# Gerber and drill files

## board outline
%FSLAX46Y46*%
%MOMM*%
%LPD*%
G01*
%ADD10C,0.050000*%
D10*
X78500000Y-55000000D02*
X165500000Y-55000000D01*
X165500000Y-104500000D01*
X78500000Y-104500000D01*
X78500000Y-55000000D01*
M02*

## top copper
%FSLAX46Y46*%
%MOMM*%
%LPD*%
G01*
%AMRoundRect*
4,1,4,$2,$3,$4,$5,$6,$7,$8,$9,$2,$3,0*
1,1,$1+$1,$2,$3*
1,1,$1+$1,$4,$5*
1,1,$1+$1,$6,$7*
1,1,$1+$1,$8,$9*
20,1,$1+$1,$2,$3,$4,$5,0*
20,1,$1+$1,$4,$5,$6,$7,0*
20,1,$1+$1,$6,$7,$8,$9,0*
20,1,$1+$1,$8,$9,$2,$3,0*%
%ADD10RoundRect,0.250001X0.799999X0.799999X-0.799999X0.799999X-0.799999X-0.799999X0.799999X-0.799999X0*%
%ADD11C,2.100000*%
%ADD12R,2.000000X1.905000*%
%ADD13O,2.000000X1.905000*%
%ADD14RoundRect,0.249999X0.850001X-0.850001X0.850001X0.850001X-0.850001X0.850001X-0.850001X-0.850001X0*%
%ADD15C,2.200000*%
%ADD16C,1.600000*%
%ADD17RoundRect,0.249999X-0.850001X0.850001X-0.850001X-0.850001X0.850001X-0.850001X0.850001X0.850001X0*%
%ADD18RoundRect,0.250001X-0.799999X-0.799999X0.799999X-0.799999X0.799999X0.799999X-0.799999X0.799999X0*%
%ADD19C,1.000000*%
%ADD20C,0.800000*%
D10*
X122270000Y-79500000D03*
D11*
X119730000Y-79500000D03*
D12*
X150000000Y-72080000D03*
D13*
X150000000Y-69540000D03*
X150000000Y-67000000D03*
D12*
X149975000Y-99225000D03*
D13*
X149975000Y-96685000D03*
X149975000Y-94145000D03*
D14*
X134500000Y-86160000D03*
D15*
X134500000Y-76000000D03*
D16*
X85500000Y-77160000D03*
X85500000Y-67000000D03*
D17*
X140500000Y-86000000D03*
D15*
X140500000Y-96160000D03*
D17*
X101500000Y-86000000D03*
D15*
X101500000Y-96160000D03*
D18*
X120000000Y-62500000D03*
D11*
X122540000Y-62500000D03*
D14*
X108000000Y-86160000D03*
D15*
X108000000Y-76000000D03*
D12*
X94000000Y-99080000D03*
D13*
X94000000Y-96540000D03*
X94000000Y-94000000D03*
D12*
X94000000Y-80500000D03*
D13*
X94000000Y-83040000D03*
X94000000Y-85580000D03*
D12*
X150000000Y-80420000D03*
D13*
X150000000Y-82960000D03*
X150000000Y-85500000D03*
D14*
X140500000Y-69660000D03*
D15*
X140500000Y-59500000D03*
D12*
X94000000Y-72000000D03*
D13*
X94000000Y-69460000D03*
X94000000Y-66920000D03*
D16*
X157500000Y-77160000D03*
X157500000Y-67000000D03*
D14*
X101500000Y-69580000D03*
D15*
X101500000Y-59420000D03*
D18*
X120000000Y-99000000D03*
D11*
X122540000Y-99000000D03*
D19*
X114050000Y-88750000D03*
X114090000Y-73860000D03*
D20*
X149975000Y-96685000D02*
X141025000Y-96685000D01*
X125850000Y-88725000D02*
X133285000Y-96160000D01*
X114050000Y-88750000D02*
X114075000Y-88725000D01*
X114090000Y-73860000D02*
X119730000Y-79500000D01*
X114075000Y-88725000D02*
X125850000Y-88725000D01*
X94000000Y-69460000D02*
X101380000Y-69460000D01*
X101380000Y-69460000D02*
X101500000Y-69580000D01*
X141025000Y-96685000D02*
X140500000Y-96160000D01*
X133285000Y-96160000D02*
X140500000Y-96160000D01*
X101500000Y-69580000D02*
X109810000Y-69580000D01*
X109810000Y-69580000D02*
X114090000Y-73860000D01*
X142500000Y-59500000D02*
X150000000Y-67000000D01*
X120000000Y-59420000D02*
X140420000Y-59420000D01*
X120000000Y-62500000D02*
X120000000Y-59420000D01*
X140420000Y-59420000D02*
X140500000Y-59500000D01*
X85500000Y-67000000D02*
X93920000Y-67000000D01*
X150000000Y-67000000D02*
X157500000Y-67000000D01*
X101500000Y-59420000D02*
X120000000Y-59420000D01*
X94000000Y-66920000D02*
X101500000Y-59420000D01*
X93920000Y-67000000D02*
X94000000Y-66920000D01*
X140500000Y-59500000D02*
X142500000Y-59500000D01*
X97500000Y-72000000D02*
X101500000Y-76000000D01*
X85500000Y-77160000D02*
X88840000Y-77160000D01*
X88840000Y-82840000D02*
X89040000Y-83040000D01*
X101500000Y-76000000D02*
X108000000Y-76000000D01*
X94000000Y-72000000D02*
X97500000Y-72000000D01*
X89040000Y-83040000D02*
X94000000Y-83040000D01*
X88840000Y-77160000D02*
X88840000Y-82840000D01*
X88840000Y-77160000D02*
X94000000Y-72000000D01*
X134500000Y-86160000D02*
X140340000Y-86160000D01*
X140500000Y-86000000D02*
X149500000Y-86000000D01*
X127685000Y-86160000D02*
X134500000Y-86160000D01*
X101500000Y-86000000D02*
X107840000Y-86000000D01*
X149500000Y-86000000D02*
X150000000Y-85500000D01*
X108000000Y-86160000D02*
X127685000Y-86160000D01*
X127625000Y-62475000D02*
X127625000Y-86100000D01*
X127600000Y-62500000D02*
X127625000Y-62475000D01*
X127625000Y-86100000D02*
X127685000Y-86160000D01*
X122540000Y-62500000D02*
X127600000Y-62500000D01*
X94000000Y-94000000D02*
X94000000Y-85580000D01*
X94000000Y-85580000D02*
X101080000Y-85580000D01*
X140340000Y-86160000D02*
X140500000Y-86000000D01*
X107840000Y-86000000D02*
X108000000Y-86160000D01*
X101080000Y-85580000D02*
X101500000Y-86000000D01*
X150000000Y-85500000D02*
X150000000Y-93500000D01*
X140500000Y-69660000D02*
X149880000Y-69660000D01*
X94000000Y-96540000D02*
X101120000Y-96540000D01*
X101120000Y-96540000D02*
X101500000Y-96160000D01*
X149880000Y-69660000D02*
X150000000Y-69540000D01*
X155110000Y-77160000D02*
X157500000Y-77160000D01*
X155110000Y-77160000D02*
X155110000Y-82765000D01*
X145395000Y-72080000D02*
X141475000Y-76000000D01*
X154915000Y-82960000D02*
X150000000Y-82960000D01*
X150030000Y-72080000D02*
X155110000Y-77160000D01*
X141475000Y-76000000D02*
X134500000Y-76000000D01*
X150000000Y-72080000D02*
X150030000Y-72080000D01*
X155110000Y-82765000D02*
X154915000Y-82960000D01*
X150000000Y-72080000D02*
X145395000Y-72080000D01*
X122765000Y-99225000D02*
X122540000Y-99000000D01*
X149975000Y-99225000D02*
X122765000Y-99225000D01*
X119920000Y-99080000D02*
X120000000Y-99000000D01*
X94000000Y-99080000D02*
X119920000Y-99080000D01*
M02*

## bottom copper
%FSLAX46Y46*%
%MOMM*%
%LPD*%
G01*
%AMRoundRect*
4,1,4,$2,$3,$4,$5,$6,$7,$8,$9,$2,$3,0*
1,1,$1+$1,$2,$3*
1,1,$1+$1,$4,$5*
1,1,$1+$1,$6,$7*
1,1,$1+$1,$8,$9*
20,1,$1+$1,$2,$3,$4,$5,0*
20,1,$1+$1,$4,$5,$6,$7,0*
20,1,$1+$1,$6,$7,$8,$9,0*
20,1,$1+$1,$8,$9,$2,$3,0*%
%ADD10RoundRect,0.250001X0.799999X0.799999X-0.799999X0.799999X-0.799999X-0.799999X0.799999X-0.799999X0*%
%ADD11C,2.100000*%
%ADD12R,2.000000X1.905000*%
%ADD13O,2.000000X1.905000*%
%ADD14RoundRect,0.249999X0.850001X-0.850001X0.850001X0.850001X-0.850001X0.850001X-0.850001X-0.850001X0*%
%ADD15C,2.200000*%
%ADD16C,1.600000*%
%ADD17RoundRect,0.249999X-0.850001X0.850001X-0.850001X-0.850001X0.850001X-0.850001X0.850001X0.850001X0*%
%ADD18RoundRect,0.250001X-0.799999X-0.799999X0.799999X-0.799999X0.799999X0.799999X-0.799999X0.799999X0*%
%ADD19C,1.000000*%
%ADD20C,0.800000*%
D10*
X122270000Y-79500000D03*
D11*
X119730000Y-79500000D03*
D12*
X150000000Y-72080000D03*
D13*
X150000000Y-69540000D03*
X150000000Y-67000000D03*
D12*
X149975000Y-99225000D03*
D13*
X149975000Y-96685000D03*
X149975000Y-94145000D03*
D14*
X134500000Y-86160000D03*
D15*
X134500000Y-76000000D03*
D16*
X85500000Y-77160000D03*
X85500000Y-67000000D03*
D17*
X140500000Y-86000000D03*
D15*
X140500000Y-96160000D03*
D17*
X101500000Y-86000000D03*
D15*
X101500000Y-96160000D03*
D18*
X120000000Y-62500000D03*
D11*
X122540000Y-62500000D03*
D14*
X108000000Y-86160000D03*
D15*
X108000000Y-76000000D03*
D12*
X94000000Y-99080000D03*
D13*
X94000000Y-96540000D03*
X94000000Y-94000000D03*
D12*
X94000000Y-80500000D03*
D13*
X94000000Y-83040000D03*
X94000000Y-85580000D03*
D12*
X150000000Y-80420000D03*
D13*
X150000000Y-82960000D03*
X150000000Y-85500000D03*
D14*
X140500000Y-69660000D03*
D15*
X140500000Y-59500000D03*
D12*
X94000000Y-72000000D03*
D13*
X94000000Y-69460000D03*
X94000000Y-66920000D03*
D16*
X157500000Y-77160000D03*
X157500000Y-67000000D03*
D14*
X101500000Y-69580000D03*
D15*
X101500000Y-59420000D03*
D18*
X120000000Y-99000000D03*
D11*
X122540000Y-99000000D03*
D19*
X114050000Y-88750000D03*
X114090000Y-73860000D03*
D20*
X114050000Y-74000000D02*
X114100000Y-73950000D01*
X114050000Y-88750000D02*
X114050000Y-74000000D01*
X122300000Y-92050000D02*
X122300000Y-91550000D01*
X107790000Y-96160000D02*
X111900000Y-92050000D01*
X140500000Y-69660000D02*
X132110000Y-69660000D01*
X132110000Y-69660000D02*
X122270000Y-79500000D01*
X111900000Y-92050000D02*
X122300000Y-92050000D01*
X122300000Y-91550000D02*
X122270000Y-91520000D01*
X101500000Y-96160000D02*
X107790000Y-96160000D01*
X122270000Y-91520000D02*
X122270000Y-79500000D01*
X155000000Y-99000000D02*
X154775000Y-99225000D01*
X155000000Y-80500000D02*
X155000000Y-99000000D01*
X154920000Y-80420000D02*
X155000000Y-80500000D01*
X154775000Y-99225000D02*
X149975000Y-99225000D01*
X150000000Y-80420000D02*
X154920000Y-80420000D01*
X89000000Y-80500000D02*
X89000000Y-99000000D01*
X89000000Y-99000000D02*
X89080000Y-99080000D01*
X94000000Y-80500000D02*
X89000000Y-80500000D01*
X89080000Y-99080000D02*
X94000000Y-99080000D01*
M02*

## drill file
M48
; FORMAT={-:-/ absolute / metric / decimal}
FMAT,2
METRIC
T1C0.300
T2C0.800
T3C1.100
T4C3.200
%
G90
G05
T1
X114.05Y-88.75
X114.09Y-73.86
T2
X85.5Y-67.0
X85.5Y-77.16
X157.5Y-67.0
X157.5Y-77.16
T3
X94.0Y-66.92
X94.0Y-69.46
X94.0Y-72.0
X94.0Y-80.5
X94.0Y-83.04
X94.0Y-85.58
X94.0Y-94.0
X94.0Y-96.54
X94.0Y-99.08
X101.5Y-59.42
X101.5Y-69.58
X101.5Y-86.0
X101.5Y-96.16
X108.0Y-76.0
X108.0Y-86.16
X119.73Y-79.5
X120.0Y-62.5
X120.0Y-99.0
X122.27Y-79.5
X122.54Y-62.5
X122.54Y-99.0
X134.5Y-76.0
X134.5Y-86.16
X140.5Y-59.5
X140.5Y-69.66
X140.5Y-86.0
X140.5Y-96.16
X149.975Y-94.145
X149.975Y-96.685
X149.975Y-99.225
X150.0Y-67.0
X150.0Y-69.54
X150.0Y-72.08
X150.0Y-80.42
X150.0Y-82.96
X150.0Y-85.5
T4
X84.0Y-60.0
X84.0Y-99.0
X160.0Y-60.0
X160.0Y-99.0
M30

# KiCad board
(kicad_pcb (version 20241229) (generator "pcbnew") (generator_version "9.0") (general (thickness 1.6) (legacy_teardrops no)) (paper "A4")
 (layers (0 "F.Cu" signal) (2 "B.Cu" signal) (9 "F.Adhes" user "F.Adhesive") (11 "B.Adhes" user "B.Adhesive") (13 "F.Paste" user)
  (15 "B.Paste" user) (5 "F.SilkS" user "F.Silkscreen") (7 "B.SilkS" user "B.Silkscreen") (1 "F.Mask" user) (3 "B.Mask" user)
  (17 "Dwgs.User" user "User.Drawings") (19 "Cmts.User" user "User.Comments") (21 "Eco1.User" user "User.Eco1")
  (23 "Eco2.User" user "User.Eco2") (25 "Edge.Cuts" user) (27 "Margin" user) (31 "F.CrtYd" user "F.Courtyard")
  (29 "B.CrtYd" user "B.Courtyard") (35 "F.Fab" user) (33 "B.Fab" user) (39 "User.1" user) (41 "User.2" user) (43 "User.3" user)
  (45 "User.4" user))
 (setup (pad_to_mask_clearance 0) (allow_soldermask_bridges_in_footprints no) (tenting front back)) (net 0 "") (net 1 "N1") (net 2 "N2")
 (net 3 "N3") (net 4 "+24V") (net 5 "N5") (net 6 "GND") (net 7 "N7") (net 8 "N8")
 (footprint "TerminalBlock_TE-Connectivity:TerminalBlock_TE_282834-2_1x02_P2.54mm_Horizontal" (layer "F.Cu") (at 122.27 79.5 180)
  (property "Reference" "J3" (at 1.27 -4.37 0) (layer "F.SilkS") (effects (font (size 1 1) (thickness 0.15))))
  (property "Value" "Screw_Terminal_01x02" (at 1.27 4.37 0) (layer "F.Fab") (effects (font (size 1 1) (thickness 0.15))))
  (pad "1" thru_hole roundrect (at 0 0 180) (size 2.1 2.1) (drill 1.1) (layers "*.Cu" "*.Mask") (remove_unused_layers no)
   (roundrect_rratio 0.119048) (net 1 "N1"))
  (pad "2" thru_hole circle (at 2.54 0 180) (size 2.1 2.1) (drill 1.1) (layers "*.Cu" "*.Mask") (remove_unused_layers no) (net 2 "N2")))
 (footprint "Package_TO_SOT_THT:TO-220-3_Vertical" (layer "F.Cu") (at 150 72.08 90)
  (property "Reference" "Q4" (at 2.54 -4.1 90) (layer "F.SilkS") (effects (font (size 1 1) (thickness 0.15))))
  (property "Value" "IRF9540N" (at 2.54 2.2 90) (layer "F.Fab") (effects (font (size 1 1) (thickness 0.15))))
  (pad "1" thru_hole rect (at 0 0 90) (size 1.905 2) (drill 1.1) (layers "*.Cu" "*.Mask") (remove_unused_layers no) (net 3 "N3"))
  (pad "2" thru_hole oval (at 2.54 0 90) (size 1.905 2) (drill 1.1) (layers "*.Cu" "*.Mask") (remove_unused_layers no) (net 1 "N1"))
  (pad "3" thru_hole oval (at 5.08 0 90) (size 1.905 2) (drill 1.1) (layers "*.Cu" "*.Mask") (remove_unused_layers no) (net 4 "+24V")))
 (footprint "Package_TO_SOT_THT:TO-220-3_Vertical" (layer "F.Cu") (at 149.975 99.225 90)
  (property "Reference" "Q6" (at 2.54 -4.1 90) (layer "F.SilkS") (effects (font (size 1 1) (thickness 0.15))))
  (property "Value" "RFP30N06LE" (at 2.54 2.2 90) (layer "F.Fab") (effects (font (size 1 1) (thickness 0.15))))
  (pad "1" thru_hole rect (at 0 0 90) (size 1.905 2) (drill 1.1) (layers "*.Cu" "*.Mask") (remove_unused_layers no) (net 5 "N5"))
  (pad "2" thru_hole oval (at 2.54 0 90) (size 1.905 2) (drill 1.1) (layers "*.Cu" "*.Mask") (remove_unused_layers no) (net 2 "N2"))
  (pad "3" thru_hole oval (at 5.08 0 90) (size 1.905 2) (drill 1.1) (layers "*.Cu" "*.Mask") (remove_unused_layers no) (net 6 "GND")))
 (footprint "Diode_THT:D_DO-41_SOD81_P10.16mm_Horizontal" (layer "F.Cu") (at 134.5 86.16 90)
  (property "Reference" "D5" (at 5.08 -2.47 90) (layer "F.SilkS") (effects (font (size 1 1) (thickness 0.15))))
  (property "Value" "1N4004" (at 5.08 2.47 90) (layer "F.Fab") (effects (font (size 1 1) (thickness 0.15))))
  (pad "1" thru_hole roundrect (at 0 0 90) (size 2.2 2.2) (drill 1.1) (layers "*.Cu" "*.Mask") (remove_unused_layers no)
   (roundrect_rratio 0.113636) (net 6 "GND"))
  (pad "2" thru_hole circle (at 10.16 0 90) (size 2.2 2.2) (drill 1.1) (layers "*.Cu" "*.Mask") (remove_unused_layers no) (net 3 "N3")))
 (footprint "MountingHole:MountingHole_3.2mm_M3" (layer "F.Cu") (at 84 99)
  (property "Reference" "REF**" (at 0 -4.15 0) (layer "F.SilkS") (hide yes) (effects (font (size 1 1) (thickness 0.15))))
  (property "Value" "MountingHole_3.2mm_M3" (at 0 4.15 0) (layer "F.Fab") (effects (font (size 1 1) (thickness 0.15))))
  (pad "" np_thru_hole circle (at 0 0) (size 3.2 3.2) (drill 3.2) (layers "*.Cu" "*.Mask")))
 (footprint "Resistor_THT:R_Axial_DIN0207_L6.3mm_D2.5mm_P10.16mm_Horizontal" (layer "F.Cu") (at 85.5 77.16 90)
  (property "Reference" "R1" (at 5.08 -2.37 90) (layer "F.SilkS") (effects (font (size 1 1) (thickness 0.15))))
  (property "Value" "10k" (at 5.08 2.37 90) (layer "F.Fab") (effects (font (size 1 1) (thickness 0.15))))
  (pad "1" thru_hole circle (at 0 0 90) (size 1.6 1.6) (drill 0.8) (layers "*.Cu" "*.Mask") (remove_unused_layers no) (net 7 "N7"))
  (pad "2" thru_hole circle (at 10.16 0 90) (size 1.6 1.6) (drill 0.8) (layers "*.Cu" "*.Mask") (remove_unused_layers no) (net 4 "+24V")))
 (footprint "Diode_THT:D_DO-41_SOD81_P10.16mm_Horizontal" (layer "F.Cu") (at 140.5 86 -90)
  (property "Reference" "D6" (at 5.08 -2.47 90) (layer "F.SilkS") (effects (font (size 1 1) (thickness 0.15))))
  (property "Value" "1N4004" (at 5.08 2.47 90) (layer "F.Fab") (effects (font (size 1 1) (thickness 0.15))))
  (pad "1" thru_hole roundrect (at 0 0 270) (size 2.2 2.2) (drill 1.1) (layers "*.Cu" "*.Mask") (remove_unused_layers no)
   (roundrect_rratio 0.113636) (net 6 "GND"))
  (pad "2" thru_hole circle (at 10.16 0 270) (size 2.2 2.2) (drill 1.1) (layers "*.Cu" "*.Mask") (remove_unused_layers no) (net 2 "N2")))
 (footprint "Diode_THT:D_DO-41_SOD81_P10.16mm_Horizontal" (layer "F.Cu") (at 101.5 86 -90)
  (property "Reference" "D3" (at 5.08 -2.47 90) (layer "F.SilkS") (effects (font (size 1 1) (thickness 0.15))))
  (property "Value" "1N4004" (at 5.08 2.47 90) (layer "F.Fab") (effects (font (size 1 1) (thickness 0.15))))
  (pad "1" thru_hole roundrect (at 0 0 270) (size 2.2 2.2) (drill 1.1) (layers "*.Cu" "*.Mask") (remove_unused_layers no)
   (roundrect_rratio 0.113636) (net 6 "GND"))
  (pad "2" thru_hole circle (at 10.16 0 270) (size 2.2 2.2) (drill 1.1) (layers "*.Cu" "*.Mask") (remove_unused_layers no) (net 1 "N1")))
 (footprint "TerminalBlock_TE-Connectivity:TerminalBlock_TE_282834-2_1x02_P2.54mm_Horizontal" (layer "F.Cu") (at 120 62.5)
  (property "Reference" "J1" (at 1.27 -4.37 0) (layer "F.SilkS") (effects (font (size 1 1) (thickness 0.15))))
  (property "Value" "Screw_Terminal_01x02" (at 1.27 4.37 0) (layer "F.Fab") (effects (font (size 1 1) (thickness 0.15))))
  (pad "1" thru_hole roundrect (at 0 0) (size 2.1 2.1) (drill 1.1) (layers "*.Cu" "*.Mask") (remove_unused_layers no)
   (roundrect_rratio 0.119048) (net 4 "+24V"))
  (pad "2" thru_hole circle (at 2.54 0) (size 2.1 2.1) (drill 1.1) (layers "*.Cu" "*.Mask") (remove_unused_layers no) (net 6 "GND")))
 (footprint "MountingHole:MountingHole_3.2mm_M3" (layer "F.Cu") (at 84 60)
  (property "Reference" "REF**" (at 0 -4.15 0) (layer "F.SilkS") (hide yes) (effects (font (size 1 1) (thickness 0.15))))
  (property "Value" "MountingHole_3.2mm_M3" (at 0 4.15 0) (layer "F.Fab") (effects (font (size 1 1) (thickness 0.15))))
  (pad "" np_thru_hole circle (at 0 0) (size 3.2 3.2) (drill 3.2) (layers "*.Cu" "*.Mask")))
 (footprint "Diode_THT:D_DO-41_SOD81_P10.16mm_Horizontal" (layer "F.Cu") (at 108 86.16 90)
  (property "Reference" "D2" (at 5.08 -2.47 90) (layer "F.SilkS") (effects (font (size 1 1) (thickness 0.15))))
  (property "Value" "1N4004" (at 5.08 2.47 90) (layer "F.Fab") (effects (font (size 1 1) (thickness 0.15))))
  (pad "1" thru_hole roundrect (at 0 0 90) (size 2.2 2.2) (drill 1.1) (layers "*.Cu" "*.Mask") (remove_unused_layers no)
   (roundrect_rratio 0.113636) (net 6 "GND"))
  (pad "2" thru_hole circle (at 10.16 0 90) (size 2.2 2.2) (drill 1.1) (layers "*.Cu" "*.Mask") (remove_unused_layers no) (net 7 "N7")))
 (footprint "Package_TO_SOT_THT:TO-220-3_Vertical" (layer "F.Cu") (at 94 99.08 90)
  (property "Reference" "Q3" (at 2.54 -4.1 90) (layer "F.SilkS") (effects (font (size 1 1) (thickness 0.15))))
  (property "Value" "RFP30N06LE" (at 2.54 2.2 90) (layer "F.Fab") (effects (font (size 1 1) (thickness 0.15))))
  (pad "1" thru_hole rect (at 0 0 90) (size 1.905 2) (drill 1.1) (layers "*.Cu" "*.Mask") (remove_unused_layers no) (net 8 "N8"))
  (pad "2" thru_hole oval (at 2.54 0 90) (size 1.905 2) (drill 1.1) (layers "*.Cu" "*.Mask") (remove_unused_layers no) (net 1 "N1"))
  (pad "3" thru_hole oval (at 5.08 0 90) (size 1.905 2) (drill 1.1) (layers "*.Cu" "*.Mask") (remove_unused_layers no) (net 6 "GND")))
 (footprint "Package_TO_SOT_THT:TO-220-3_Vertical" (layer "F.Cu") (at 94 80.5 -90)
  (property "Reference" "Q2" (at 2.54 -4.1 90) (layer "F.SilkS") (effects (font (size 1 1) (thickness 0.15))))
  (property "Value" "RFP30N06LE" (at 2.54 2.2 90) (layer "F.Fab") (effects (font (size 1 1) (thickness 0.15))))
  (pad "1" thru_hole rect (at 0 0 270) (size 1.905 2) (drill 1.1) (layers "*.Cu" "*.Mask") (remove_unused_layers no) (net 8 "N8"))
  (pad "2" thru_hole oval (at 2.54 0 270) (size 1.905 2) (drill 1.1) (layers "*.Cu" "*.Mask") (remove_unused_layers no) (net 7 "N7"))
  (pad "3" thru_hole oval (at 5.08 0 270) (size 1.905 2) (drill 1.1) (layers "*.Cu" "*.Mask") (remove_unused_layers no) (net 6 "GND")))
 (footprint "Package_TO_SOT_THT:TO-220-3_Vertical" (layer "F.Cu") (at 150 80.42 -90)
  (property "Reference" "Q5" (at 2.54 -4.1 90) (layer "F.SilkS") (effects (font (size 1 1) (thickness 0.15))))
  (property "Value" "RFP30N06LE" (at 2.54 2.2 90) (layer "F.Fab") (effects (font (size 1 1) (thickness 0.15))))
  (pad "1" thru_hole rect (at 0 0 270) (size 1.905 2) (drill 1.1) (layers "*.Cu" "*.Mask") (remove_unused_layers no) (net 5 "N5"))
  (pad "2" thru_hole oval (at 2.54 0 270) (size 1.905 2) (drill 1.1) (layers "*.Cu" "*.Mask") (remove_unused_layers no) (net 3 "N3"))
  (pad "3" thru_hole oval (at 5.08 0 270) (size 1.905 2) (drill 1.1) (layers "*.Cu" "*.Mask") (remove_unused_layers no) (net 6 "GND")))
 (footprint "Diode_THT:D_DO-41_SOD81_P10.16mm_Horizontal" (layer "F.Cu") (at 140.5 69.66 90)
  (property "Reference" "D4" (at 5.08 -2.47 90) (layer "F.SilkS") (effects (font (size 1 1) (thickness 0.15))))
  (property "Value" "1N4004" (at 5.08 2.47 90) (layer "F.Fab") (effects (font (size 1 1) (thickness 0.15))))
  (pad "1" thru_hole roundrect (at 0 0 90) (size 2.2 2.2) (drill 1.1) (layers "*.Cu" "*.Mask") (remove_unused_layers no)
   (roundrect_rratio 0.113636) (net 1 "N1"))
  (pad "2" thru_hole circle (at 10.16 0 90) (size 2.2 2.2) (drill 1.1) (layers "*.Cu" "*.Mask") (remove_unused_layers no) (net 4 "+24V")))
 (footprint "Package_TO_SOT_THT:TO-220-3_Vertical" (layer "F.Cu") (at 94 72 90)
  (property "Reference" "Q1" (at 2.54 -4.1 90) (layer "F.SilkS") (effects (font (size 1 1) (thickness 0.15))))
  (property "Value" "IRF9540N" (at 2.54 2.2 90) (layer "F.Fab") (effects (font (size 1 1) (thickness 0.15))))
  (pad "1" thru_hole rect (at 0 0 90) (size 1.905 2) (drill 1.1) (layers "*.Cu" "*.Mask") (remove_unused_layers no) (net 7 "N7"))
  (pad "2" thru_hole oval (at 2.54 0 90) (size 1.905 2) (drill 1.1) (layers "*.Cu" "*.Mask") (remove_unused_layers no) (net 2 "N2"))
  (pad "3" thru_hole oval (at 5.08 0 90) (size 1.905 2) (drill 1.1) (layers "*.Cu" "*.Mask") (remove_unused_layers no) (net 4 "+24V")))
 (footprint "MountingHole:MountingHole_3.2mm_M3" (layer "F.Cu") (at 160 60)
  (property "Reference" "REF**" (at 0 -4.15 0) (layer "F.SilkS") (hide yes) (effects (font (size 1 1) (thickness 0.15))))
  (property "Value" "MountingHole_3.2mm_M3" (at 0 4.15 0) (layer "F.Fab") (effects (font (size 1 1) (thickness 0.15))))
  (pad "" np_thru_hole circle (at 0 0) (size 3.2 3.2) (drill 3.2) (layers "*.Cu" "*.Mask")))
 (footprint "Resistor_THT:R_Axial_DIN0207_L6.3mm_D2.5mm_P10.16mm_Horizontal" (layer "F.Cu") (at 157.5 77.16 90)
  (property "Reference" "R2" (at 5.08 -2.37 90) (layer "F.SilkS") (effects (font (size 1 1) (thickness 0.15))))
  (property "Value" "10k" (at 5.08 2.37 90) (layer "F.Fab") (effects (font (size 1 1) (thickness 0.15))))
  (pad "1" thru_hole circle (at 0 0 90) (size 1.6 1.6) (drill 0.8) (layers "*.Cu" "*.Mask") (remove_unused_layers no) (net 3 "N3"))
  (pad "2" thru_hole circle (at 10.16 0 90) (size 1.6 1.6) (drill 0.8) (layers "*.Cu" "*.Mask") (remove_unused_layers no) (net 4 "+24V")))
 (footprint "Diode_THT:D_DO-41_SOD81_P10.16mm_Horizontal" (layer "F.Cu") (at 101.5 69.58 90)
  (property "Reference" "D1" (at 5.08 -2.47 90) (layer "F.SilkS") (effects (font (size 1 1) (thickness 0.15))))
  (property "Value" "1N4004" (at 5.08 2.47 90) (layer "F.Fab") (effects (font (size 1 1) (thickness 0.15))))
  (pad "1" thru_hole roundrect (at 0 0 90) (size 2.2 2.2) (drill 1.1) (layers "*.Cu" "*.Mask") (remove_unused_layers no)
   (roundrect_rratio 0.113636) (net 2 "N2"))
  (pad "2" thru_hole circle (at 10.16 0 90) (size 2.2 2.2) (drill 1.1) (layers "*.Cu" "*.Mask") (remove_unused_layers no) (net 4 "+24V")))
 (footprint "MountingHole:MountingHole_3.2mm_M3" (layer "F.Cu") (at 160 99)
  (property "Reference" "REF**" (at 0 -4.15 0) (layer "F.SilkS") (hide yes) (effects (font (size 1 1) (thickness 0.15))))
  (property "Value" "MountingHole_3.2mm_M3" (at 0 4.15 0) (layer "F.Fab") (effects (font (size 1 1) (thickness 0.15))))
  (pad "" np_thru_hole circle (at 0 0) (size 3.2 3.2) (drill 3.2) (layers "*.Cu" "*.Mask")))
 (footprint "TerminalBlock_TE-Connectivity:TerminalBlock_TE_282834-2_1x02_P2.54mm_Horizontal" (layer "F.Cu") (at 120 99)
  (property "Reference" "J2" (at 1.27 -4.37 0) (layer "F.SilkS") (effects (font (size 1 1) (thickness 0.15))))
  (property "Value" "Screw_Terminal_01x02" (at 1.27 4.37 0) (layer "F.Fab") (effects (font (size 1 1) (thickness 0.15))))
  (pad "1" thru_hole roundrect (at 0 0) (size 2.1 2.1) (drill 1.1) (layers "*.Cu" "*.Mask") (remove_unused_layers no)
   (roundrect_rratio 0.119048) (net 8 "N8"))
  (pad "2" thru_hole circle (at 2.54 0) (size 2.1 2.1) (drill 1.1) (layers "*.Cu" "*.Mask") (remove_unused_layers no) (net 5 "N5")))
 (gr_rect (start 78.5 55) (end 165.5 104.5) (stroke (width 0.05) (type default)) (fill no) (layer "Edge.Cuts"))
 (segment (start 149.975 96.685) (end 141.025 96.685) (width 0.8) (layer "F.Cu") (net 2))
 (segment (start 125.85 88.725) (end 133.285 96.16) (width 0.8) (layer "F.Cu") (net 2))
 (segment (start 114.05 88.75) (end 114.075 88.725) (width 0.8) (layer "F.Cu") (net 2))
 (segment (start 114.09 73.86) (end 119.73 79.5) (width 0.8) (layer "F.Cu") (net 2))
 (segment (start 114.075 88.725) (end 125.85 88.725) (width 0.8) (layer "F.Cu") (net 2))
 (segment (start 94 69.46) (end 101.38 69.46) (width 0.8) (layer "F.Cu") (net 2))
 (segment (start 101.38 69.46) (end 101.5 69.58) (width 0.8) (layer "F.Cu") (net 2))
 (segment (start 141.025 96.685) (end 140.5 96.16) (width 0.8) (layer "F.Cu") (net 2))
 (segment (start 133.285 96.16) (end 140.5 96.16) (width 0.8) (layer "F.Cu") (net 2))
 (segment (start 101.5 69.58) (end 109.81 69.58) (width 0.8) (layer "F.Cu") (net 2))
 (segment (start 109.81 69.58) (end 114.09 73.86) (width 0.8) (layer "F.Cu") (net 2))
 (via (at 114.05 88.75) (size 1) (drill 0.3) (layers "F.Cu" "B.Cu") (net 2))
 (via (at 114.09 73.86) (size 1) (drill 0.3) (layers "F.Cu" "B.Cu") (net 2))
 (segment (start 114.05 74) (end 114.1 73.95) (width 0.8) (layer "B.Cu") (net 2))
 (segment (start 114.05 88.75) (end 114.05 74) (width 0.8) (layer "B.Cu") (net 2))
 (segment (start 142.5 59.5) (end 150 67) (width 0.8) (layer "F.Cu") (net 4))
 (segment (start 120 59.42) (end 140.42 59.42) (width 0.8) (layer "F.Cu") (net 4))
 (segment (start 120 62.5) (end 120 59.42) (width 0.8) (layer "F.Cu") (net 4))
 (segment (start 140.42 59.42) (end 140.5 59.5) (width 0.8) (layer "F.Cu") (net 4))
 (segment (start 85.5 67) (end 93.92 67) (width 0.8) (layer "F.Cu") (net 4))
 (segment (start 150 67) (end 157.5 67) (width 0.8) (layer "F.Cu") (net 4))
 (segment (start 101.5 59.42) (end 120 59.42) (width 0.8) (layer "F.Cu") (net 4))
 (segment (start 94 66.92) (end 101.5 59.42) (width 0.8) (layer "F.Cu") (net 4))
 (segment (start 93.92 67) (end 94 66.92) (width 0.8) (layer "F.Cu") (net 4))
 (segment (start 140.5 59.5) (end 142.5 59.5) (width 0.8) (layer "F.Cu") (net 4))
 (segment (start 97.5 72) (end 101.5 76) (width 0.8) (layer "F.Cu") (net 7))
 (segment (start 85.5 77.16) (end 88.84 77.16) (width 0.8) (layer "F.Cu") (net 7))
 (segment (start 88.84 82.84) (end 89.04 83.04) (width 0.8) (layer "F.Cu") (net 7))
 (segment (start 101.5 76) (end 108 76) (width 0.8) (layer "F.Cu") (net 7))
 (segment (start 94 72) (end 97.5 72) (width 0.8) (layer "F.Cu") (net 7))
 (segment (start 89.04 83.04) (end 94 83.04) (width 0.8) (layer "F.Cu") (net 7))
 (segment (start 88.84 77.16) (end 88.84 82.84) (width 0.8) (layer "F.Cu") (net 7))
 (segment (start 88.84 77.16) (end 94 72) (width 0.8) (layer "F.Cu") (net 7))
 (segment (start 134.5 86.16) (end 140.34 86.16) (width 0.8) (layer "F.Cu") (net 6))
 (segment (start 140.5 86) (end 149.5 86) (width 0.8) (layer "F.Cu") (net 6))
 (segment (start 127.685 86.16) (end 134.5 86.16) (width 0.8) (layer "F.Cu") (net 6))
 (segment (start 101.5 86) (end 107.84 86) (width 0.8) (layer "F.Cu") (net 6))
 (segment (start 149.5 86) (end 150 85.5) (width 0.8) (layer "F.Cu") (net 6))
 (segment (start 108 86.16) (end 127.685 86.16) (width 0.8) (layer "F.Cu") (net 6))
 (segment (start 127.625 62.475) (end 127.625 86.1) (width 0.8) (layer "F.Cu") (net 6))
 (segment (start 127.6 62.5) (end 127.625 62.475) (width 0.8) (layer "F.Cu") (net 6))
 (segment (start 127.625 86.1) (end 127.685 86.16) (width 0.8) (layer "F.Cu") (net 6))
 (segment (start 122.54 62.5) (end 127.6 62.5) (width 0.8) (layer "F.Cu") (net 6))
 (segment (start 94 94) (end 94 85.58) (width 0.8) (layer "F.Cu") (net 6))
 (segment (start 94 85.58) (end 101.08 85.58) (width 0.8) (layer "F.Cu") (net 6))
 (segment (start 140.34 86.16) (end 140.5 86) (width 0.8) (layer "F.Cu") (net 6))
 (segment (start 107.84 86) (end 108 86.16) (width 0.8) (layer "F.Cu") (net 6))
 (segment (start 101.08 85.58) (end 101.5 86) (width 0.8) (layer "F.Cu") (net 6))
 (segment (start 150 85.5) (end 150 93.5) (width 0.8) (layer "F.Cu") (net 6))
 (segment (start 140.5 69.66) (end 149.88 69.66) (width 0.8) (layer "F.Cu") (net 1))
 (segment (start 94 96.54) (end 101.12 96.54) (width 0.8) (layer "F.Cu") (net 1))
 (segment (start 101.12 96.54) (end 101.5 96.16) (width 0.8) (layer "F.Cu") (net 1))
 (segment (start 149.88 69.66) (end 150 69.54) (width 0.8) (layer "F.Cu") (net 1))
 (segment (start 122.3 92.05) (end 122.3 91.55) (width 0.8) (layer "B.Cu") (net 1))
 (segment (start 107.79 96.16) (end 111.9 92.05) (width 0.8) (layer "B.Cu") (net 1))
 (segment (start 140.5 69.66) (end 132.11 69.66) (width 0.8) (layer "B.Cu") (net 1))
 (segment (start 132.11 69.66) (end 122.27 79.5) (width 0.8) (layer "B.Cu") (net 1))
 (segment (start 111.9 92.05) (end 122.3 92.05) (width 0.8) (layer "B.Cu") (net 1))
 (segment (start 122.3 91.55) (end 122.27 91.52) (width 0.8) (layer "B.Cu") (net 1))
 (segment (start 101.5 96.16) (end 107.79 96.16) (width 0.8) (layer "B.Cu") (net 1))
 (segment (start 122.27 91.52) (end 122.27 79.5) (width 0.8) (layer "B.Cu") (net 1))
 (segment (start 155.11 77.16) (end 157.5 77.16) (width 0.8) (layer "F.Cu") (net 3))
 (segment (start 155.11 77.16) (end 155.11 82.765) (width 0.8) (layer "F.Cu") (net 3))
 (segment (start 145.395 72.08) (end 141.475 76) (width 0.8) (layer "F.Cu") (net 3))
 (segment (start 154.915 82.96) (end 150 82.96) (width 0.8) (layer "F.Cu") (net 3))
 (segment (start 150.03 72.08) (end 155.11 77.16) (width 0.8) (layer "F.Cu") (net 3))
 (segment (start 141.475 76) (end 134.5 76) (width 0.8) (layer "F.Cu") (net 3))
 (segment (start 150 72.08) (end 150.03 72.08) (width 0.8) (layer "F.Cu") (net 3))
 (segment (start 155.11 82.765) (end 154.915 82.96) (width 0.8) (layer "F.Cu") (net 3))
 (segment (start 150 72.08) (end 145.395 72.08) (width 0.8) (layer "F.Cu") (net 3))
 (segment (start 122.765 99.225) (end 122.54 99) (width 0.8) (layer "F.Cu") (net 5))
 (segment (start 149.975 99.225) (end 122.765 99.225) (width 0.8) (layer "F.Cu") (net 5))
 (segment (start 155 99) (end 154.775 99.225) (width 0.8) (layer "B.Cu") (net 5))
 (segment (start 155 80.5) (end 155 99) (width 0.8) (layer "B.Cu") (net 5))
 (segment (start 154.92 80.42) (end 155 80.5) (width 0.8) (layer "B.Cu") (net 5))
 (segment (start 154.775 99.225) (end 149.975 99.225) (width 0.8) (layer "B.Cu") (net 5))
 (segment (start 150 80.42) (end 154.92 80.42) (width 0.8) (layer "B.Cu") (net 5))
 (segment (start 119.92 99.08) (end 120 99) (width 0.8) (layer "F.Cu") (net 8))
 (segment (start 94 99.08) (end 119.92 99.08) (width 0.8) (layer "F.Cu") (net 8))
 (segment (start 89 80.5) (end 89 99) (width 0.8) (layer "B.Cu") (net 8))
 (segment (start 89 99) (end 89.08 99.08) (width 0.8) (layer "B.Cu") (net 8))
 (segment (start 94 80.5) (end 89 80.5) (width 0.8) (layer "B.Cu") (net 8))
 (segment (start 89.08 99.08) (end 94 99.08) (width 0.8) (layer "B.Cu") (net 8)))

